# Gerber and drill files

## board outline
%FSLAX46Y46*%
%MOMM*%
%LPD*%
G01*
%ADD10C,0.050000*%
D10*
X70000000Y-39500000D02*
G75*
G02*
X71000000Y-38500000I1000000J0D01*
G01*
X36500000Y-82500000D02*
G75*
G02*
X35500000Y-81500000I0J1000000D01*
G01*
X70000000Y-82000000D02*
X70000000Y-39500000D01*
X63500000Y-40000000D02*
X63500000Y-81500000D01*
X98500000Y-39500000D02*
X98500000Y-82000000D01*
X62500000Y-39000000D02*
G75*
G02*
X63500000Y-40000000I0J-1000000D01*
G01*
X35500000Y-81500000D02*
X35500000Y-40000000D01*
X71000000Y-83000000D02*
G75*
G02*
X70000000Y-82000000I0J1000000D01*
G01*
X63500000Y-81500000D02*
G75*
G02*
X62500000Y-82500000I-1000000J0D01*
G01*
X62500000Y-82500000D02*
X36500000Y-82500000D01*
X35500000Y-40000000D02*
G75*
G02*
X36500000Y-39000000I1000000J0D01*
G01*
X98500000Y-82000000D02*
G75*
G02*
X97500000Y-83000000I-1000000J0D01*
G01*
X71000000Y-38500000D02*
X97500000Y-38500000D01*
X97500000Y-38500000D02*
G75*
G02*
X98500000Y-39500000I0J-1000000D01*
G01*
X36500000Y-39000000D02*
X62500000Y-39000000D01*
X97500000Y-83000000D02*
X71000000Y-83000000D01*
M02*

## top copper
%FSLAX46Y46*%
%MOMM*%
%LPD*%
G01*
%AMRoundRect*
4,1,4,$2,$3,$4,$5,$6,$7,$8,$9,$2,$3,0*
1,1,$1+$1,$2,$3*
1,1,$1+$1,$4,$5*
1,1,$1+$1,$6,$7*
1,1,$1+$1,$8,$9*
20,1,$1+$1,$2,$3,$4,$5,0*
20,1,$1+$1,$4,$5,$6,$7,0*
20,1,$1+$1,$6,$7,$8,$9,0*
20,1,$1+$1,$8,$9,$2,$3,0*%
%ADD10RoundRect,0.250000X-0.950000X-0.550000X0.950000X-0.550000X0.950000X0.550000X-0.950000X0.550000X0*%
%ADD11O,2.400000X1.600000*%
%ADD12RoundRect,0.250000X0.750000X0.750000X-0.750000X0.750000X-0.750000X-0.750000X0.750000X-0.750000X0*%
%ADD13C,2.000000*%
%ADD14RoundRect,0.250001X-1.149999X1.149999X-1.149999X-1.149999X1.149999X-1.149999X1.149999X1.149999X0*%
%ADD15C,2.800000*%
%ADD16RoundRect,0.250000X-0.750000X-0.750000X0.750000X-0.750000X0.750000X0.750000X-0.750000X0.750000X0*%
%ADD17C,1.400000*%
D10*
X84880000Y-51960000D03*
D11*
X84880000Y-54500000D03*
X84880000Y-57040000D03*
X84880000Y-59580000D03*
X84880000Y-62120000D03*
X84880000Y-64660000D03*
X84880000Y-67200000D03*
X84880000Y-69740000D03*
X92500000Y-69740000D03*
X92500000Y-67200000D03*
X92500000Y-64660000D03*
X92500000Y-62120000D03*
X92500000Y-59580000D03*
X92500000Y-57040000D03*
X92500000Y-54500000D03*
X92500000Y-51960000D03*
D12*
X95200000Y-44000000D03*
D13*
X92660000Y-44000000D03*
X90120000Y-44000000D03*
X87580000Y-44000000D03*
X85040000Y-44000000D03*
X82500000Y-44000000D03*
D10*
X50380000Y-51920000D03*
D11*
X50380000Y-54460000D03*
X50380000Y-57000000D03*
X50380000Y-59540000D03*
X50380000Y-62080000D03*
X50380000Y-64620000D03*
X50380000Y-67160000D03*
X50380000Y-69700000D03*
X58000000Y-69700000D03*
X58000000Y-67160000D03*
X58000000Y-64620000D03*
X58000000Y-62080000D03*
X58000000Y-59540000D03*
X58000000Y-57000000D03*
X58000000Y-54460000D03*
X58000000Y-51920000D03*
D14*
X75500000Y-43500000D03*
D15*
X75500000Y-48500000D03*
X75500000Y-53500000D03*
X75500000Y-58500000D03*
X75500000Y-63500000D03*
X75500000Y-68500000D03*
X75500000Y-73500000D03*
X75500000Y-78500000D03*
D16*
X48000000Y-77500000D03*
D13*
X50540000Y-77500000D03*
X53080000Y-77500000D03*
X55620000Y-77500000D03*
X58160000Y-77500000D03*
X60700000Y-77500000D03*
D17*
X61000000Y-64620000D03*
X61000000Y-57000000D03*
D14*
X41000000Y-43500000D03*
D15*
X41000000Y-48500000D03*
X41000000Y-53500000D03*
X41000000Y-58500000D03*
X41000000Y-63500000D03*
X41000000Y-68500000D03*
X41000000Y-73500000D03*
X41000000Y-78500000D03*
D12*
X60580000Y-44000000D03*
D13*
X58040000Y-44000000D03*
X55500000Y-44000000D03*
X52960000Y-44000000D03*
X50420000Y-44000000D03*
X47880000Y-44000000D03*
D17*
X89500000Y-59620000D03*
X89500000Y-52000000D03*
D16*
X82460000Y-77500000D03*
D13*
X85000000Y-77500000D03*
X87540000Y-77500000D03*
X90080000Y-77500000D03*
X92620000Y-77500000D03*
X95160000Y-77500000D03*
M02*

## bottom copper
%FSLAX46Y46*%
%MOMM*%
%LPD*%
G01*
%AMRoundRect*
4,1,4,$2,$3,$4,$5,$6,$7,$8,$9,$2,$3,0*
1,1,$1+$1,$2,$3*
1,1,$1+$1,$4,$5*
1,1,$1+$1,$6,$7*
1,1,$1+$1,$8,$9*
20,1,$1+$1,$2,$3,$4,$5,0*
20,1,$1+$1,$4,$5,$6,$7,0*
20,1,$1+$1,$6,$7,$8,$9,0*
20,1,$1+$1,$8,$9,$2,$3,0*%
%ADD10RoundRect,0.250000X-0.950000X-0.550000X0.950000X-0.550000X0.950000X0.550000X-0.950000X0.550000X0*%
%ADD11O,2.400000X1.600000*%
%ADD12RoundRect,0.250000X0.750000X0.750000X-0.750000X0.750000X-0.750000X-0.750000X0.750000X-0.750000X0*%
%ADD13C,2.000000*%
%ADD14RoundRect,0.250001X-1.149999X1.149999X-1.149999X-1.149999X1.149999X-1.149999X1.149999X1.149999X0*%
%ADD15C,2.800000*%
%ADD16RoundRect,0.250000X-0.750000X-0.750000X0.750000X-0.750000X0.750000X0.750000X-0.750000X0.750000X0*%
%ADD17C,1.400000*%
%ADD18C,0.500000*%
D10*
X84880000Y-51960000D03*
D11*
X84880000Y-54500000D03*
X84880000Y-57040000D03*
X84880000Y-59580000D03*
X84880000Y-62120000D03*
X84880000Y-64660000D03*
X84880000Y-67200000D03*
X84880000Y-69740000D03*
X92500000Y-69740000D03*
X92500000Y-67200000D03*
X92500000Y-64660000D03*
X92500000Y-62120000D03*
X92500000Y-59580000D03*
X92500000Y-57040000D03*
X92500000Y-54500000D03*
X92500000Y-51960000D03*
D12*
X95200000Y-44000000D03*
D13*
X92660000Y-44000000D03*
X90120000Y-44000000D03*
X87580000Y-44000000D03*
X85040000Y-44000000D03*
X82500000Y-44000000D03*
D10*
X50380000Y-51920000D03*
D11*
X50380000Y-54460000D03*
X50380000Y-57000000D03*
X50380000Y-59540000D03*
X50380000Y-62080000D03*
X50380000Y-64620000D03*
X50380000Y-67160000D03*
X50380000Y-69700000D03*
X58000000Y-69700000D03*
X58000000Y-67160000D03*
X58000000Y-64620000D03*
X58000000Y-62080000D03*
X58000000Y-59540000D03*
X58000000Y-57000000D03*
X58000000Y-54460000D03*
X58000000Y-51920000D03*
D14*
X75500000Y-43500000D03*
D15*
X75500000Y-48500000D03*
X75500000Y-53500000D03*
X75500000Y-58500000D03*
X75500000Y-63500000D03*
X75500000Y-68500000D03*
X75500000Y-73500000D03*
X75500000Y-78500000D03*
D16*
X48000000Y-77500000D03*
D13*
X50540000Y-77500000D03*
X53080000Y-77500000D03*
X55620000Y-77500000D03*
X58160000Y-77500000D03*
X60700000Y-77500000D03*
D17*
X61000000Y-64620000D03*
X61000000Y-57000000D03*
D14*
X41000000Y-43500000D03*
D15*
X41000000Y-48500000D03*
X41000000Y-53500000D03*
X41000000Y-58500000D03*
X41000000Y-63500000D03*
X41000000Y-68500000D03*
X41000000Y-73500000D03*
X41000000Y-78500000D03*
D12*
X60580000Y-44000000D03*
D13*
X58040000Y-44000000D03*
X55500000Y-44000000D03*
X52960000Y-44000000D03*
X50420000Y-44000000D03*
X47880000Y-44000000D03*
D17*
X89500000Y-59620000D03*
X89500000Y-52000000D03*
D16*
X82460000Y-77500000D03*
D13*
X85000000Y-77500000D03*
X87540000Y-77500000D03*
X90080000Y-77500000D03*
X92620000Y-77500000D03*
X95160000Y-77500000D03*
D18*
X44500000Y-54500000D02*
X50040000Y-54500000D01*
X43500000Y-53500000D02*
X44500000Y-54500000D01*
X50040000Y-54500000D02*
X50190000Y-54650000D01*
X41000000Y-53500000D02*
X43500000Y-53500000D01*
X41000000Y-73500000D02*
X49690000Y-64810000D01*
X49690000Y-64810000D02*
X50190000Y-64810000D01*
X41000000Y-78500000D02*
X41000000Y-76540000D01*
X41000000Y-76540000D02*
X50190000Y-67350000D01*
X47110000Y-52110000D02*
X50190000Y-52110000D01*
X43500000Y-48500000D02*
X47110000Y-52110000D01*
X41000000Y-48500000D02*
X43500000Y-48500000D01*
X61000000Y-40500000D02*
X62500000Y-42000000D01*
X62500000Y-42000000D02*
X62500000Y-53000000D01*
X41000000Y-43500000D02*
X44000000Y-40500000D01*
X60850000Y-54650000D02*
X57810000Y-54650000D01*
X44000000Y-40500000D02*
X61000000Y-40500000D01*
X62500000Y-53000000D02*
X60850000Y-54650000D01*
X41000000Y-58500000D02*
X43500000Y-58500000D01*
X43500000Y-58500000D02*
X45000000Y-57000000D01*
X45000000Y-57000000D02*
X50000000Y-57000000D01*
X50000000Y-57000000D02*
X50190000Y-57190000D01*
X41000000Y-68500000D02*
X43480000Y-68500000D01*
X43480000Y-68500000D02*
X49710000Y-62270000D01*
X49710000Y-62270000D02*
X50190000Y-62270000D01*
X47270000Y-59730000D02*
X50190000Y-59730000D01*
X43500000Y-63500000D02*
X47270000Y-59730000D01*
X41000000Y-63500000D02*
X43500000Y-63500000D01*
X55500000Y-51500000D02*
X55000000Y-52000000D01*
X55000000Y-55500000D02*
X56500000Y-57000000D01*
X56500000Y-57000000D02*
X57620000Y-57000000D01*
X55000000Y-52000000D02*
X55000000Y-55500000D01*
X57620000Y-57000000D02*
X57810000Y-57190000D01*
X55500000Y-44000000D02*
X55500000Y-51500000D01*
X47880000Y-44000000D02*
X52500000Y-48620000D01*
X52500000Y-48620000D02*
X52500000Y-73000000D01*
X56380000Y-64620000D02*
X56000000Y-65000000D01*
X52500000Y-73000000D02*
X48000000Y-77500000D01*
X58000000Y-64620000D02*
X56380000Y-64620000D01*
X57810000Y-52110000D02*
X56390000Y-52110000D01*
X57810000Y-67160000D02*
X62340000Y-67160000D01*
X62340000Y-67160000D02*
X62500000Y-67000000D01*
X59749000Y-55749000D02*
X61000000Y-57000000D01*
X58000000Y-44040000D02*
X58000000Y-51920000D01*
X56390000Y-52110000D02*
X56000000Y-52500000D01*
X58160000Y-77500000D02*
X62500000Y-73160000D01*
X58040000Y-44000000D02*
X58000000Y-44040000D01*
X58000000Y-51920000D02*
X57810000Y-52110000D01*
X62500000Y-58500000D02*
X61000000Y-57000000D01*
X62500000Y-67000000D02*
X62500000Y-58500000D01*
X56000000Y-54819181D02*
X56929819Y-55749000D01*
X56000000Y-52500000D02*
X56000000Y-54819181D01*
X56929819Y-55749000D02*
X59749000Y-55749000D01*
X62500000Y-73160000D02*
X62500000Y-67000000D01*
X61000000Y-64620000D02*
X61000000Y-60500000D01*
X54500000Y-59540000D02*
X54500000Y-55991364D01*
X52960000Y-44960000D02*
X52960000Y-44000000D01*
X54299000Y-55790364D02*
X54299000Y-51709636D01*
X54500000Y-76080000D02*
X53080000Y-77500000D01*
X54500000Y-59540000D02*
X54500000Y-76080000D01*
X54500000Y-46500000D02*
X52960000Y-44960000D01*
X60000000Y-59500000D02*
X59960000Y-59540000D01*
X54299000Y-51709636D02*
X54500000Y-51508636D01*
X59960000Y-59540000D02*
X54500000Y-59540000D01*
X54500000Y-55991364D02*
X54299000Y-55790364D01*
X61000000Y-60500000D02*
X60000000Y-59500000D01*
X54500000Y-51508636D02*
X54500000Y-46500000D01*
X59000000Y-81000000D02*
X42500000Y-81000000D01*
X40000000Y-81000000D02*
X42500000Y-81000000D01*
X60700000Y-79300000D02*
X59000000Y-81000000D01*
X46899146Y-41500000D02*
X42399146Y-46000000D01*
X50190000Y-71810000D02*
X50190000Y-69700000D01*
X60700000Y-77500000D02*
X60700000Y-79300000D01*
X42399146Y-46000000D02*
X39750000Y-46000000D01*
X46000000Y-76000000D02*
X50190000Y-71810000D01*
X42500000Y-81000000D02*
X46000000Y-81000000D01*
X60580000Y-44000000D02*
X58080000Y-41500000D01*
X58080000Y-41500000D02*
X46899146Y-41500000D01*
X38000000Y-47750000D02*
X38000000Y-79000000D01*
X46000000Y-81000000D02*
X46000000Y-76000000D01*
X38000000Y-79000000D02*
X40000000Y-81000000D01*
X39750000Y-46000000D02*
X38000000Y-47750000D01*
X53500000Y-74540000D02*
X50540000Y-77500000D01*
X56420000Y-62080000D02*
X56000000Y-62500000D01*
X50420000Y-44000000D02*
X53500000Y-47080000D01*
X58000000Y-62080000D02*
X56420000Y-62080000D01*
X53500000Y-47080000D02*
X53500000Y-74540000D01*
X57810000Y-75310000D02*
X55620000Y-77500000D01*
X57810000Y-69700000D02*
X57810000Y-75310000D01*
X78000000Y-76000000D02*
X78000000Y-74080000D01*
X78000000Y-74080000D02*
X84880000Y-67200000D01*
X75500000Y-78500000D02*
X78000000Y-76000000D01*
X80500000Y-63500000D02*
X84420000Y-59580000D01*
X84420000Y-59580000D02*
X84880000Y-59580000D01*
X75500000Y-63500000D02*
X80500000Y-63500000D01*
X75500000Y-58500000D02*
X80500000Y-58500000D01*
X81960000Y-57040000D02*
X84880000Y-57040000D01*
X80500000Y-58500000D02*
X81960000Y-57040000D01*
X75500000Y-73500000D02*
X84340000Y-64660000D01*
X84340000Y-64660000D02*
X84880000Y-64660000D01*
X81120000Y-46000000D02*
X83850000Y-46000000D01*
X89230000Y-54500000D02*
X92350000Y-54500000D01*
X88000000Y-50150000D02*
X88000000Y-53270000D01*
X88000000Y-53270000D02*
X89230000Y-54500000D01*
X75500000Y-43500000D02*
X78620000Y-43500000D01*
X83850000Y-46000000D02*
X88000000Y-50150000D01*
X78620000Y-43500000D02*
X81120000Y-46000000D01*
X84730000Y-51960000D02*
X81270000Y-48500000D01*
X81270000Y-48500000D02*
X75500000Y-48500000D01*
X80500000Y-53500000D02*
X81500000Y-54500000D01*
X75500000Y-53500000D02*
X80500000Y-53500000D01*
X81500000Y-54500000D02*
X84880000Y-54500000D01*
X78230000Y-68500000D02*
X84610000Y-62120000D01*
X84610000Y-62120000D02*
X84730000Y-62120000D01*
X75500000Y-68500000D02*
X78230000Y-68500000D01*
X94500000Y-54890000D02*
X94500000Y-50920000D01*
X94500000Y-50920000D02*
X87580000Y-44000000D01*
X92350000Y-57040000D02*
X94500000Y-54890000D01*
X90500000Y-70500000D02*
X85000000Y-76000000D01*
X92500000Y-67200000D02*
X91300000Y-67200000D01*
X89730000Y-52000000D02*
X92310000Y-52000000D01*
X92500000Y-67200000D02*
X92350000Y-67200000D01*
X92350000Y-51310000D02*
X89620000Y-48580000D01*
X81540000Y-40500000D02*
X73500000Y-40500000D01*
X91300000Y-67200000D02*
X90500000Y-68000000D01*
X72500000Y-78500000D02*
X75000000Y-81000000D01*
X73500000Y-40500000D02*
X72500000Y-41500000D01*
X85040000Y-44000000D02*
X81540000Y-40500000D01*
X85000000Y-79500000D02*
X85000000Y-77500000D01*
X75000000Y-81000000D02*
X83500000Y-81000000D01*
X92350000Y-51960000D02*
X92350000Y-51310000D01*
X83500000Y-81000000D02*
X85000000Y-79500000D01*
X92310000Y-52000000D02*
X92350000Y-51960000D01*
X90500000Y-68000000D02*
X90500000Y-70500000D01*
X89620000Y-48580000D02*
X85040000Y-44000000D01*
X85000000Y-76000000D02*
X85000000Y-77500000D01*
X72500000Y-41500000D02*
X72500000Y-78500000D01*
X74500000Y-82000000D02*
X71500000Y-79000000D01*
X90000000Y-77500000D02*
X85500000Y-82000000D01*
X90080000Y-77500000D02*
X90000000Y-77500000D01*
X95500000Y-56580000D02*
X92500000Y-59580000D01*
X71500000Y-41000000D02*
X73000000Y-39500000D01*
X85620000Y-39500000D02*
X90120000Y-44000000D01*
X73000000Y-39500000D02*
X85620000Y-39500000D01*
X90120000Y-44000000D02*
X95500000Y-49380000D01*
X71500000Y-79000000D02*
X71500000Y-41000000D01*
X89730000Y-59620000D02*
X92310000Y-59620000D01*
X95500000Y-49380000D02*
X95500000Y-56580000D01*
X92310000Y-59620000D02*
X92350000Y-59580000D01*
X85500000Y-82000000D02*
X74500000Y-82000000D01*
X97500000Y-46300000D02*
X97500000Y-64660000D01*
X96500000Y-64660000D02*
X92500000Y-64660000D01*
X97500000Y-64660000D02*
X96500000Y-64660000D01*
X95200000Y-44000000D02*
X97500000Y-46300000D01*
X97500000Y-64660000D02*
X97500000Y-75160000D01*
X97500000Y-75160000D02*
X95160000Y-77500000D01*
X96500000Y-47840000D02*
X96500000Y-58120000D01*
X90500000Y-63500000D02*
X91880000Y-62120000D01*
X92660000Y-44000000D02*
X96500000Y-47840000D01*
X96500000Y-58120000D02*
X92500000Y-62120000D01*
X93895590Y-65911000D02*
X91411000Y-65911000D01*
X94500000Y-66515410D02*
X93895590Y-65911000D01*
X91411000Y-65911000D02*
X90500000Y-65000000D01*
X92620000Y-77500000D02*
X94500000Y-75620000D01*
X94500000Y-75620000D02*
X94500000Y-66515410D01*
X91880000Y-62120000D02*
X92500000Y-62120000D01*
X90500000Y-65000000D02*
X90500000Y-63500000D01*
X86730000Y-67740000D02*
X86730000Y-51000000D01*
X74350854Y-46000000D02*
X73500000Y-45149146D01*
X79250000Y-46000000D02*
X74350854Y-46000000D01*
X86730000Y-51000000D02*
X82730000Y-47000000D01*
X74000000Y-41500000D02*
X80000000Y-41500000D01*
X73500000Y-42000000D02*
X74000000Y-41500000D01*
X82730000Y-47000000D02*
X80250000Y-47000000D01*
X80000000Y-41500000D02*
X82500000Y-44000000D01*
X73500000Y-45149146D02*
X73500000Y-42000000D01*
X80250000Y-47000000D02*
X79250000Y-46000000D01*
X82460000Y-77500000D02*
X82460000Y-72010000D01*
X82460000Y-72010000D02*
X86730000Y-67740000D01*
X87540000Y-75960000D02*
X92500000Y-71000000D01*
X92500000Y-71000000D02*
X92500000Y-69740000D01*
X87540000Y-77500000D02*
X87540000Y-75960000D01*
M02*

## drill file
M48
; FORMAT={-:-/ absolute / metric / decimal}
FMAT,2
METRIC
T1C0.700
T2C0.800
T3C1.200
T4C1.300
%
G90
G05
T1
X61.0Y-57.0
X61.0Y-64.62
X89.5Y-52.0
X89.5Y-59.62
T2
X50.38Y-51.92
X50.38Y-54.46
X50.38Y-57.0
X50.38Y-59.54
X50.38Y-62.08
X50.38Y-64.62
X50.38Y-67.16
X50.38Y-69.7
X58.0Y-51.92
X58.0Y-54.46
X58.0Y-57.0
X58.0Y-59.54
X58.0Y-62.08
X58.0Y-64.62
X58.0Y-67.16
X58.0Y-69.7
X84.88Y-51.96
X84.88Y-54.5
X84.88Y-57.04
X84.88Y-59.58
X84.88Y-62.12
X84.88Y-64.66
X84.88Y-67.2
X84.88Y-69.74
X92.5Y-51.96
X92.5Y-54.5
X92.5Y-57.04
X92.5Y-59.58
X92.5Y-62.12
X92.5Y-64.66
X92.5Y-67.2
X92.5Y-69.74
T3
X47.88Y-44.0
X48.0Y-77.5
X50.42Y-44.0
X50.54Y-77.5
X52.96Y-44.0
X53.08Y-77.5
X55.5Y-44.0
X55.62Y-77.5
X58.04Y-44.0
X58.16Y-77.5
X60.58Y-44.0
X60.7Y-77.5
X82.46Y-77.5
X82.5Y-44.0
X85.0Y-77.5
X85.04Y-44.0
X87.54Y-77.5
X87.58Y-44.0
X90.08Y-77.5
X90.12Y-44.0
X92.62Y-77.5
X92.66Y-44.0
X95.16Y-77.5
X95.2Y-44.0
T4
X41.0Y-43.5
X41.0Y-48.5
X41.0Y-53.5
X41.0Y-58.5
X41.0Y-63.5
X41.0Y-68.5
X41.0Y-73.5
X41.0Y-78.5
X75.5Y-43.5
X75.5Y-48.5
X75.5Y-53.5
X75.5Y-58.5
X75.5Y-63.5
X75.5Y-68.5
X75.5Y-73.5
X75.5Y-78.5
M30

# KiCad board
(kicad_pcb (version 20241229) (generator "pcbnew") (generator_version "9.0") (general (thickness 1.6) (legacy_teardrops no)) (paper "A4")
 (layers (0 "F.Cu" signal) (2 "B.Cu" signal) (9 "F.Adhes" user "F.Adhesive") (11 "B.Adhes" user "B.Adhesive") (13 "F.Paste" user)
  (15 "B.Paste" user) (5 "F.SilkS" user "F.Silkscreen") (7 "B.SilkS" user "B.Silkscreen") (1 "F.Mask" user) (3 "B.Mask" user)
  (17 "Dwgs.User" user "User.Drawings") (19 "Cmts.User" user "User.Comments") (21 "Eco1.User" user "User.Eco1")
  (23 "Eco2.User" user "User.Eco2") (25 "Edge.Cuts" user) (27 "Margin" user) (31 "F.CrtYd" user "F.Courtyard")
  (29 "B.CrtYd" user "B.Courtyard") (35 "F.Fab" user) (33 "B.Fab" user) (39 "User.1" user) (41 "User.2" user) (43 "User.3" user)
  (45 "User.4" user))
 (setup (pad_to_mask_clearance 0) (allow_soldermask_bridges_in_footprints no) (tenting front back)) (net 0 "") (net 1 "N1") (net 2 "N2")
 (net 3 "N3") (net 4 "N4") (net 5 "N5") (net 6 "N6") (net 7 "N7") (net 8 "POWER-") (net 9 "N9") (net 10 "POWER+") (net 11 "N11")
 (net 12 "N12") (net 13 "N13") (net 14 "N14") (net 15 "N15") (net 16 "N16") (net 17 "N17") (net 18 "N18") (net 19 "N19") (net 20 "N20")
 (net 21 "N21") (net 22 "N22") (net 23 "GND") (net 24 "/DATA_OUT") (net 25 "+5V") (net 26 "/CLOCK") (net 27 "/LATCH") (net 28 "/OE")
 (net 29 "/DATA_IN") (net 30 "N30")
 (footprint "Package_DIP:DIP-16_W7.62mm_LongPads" (layer "F.Cu") (at 84.88 51.96)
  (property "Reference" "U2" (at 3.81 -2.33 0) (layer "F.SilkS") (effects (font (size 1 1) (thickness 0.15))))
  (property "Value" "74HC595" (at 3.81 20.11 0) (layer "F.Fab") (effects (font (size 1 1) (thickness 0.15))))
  (pad "1" thru_hole roundrect (at 0 0) (size 2.4 1.6) (drill 0.8) (layers "*.Cu" "*.Mask") (remove_unused_layers no)
   (roundrect_rratio 0.15625) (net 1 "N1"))
  (pad "2" thru_hole oval (at 0 2.54) (size 2.4 1.6) (drill 0.8) (layers "*.Cu" "*.Mask") (remove_unused_layers no) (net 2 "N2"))
  (pad "3" thru_hole oval (at 0 5.08) (size 2.4 1.6) (drill 0.8) (layers "*.Cu" "*.Mask") (remove_unused_layers no) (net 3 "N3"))
  (pad "4" thru_hole oval (at 0 7.62) (size 2.4 1.6) (drill 0.8) (layers "*.Cu" "*.Mask") (remove_unused_layers no) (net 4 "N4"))
  (pad "5" thru_hole oval (at 0 10.16) (size 2.4 1.6) (drill 0.8) (layers "*.Cu" "*.Mask") (remove_unused_layers no) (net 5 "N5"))
  (pad "6" thru_hole oval (at 0 12.7) (size 2.4 1.6) (drill 0.8) (layers "*.Cu" "*.Mask") (remove_unused_layers no) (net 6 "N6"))
  (pad "7" thru_hole oval (at 0 15.24) (size 2.4 1.6) (drill 0.8) (layers "*.Cu" "*.Mask") (remove_unused_layers no) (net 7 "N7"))
  (pad "8" thru_hole oval (at 0 17.78) (size 2.4 1.6) (drill 0.8) (layers "*.Cu" "*.Mask") (remove_unused_layers no) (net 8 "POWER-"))
  (pad "9" thru_hole oval (at 7.62 17.78) (size 2.4 1.6) (drill 0.8) (layers "*.Cu" "*.Mask") (remove_unused_layers no) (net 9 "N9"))
  (pad "10" thru_hole oval (at 7.62 15.24) (size 2.4 1.6) (drill 0.8) (layers "*.Cu" "*.Mask") (remove_unused_layers no) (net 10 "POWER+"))
  (pad "11" thru_hole oval (at 7.62 12.7) (size 2.4 1.6) (drill 0.8) (layers "*.Cu" "*.Mask") (remove_unused_layers no) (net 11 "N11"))
  (pad "12" thru_hole oval (at 7.62 10.16) (size 2.4 1.6) (drill 0.8) (layers "*.Cu" "*.Mask") (remove_unused_layers no) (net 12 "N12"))
  (pad "13" thru_hole oval (at 7.62 7.62) (size 2.4 1.6) (drill 0.8) (layers "*.Cu" "*.Mask") (remove_unused_layers no) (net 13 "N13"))
  (pad "14" thru_hole oval (at 7.62 5.08) (size 2.4 1.6) (drill 0.8) (layers "*.Cu" "*.Mask") (remove_unused_layers no) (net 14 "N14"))
  (pad "15" thru_hole oval (at 7.62 2.54) (size 2.4 1.6) (drill 0.8) (layers "*.Cu" "*.Mask") (remove_unused_layers no) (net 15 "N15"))
  (pad "16" thru_hole oval (at 7.62 0) (size 2.4 1.6) (drill 0.8) (layers "*.Cu" "*.Mask") (remove_unused_layers no) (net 10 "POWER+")))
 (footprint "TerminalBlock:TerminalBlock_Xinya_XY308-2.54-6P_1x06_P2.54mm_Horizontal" (layer "F.Cu") (at 95.2 44 180)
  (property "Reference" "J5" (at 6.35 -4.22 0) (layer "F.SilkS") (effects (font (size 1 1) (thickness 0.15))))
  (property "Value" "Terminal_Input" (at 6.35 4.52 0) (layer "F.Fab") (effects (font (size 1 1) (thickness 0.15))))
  (pad "1" thru_hole roundrect (at 0 0 180) (size 2 2) (drill 1.2) (layers "*.Cu" "*.Mask") (remove_unused_layers no)
   (roundrect_rratio 0.125) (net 11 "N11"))
  (pad "2" thru_hole circle (at 2.54 0 180) (size 2 2) (drill 1.2) (layers "*.Cu" "*.Mask") (remove_unused_layers no) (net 12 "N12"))
  (pad "3" thru_hole circle (at 5.08 0 180) (size 2 2) (drill 1.2) (layers "*.Cu" "*.Mask") (remove_unused_layers no) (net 13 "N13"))
  (pad "4" thru_hole circle (at 7.62 0 180) (size 2 2) (drill 1.2) (layers "*.Cu" "*.Mask") (remove_unused_layers no) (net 14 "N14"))
  (pad "5" thru_hole circle (at 10.16 0 180) (size 2 2) (drill 1.2) (layers "*.Cu" "*.Mask") (remove_unused_layers no) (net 10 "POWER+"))
  (pad "6" thru_hole circle (at 12.7 0 180) (size 2 2) (drill 1.2) (layers "*.Cu" "*.Mask") (remove_unused_layers no) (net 8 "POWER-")))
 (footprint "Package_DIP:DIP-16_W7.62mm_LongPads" (layer "F.Cu") (at 50.38 51.92)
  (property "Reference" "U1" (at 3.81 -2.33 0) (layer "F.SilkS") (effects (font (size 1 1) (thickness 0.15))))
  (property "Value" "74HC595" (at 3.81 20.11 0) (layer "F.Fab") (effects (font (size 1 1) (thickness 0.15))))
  (pad "1" thru_hole roundrect (at 0 0) (size 2.4 1.6) (drill 0.8) (layers "*.Cu" "*.Mask") (remove_unused_layers no)
   (roundrect_rratio 0.15625) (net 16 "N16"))
  (pad "2" thru_hole oval (at 0 2.54) (size 2.4 1.6) (drill 0.8) (layers "*.Cu" "*.Mask") (remove_unused_layers no) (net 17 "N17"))
  (pad "3" thru_hole oval (at 0 5.08) (size 2.4 1.6) (drill 0.8) (layers "*.Cu" "*.Mask") (remove_unused_layers no) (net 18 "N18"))
  (pad "4" thru_hole oval (at 0 7.62) (size 2.4 1.6) (drill 0.8) (layers "*.Cu" "*.Mask") (remove_unused_layers no) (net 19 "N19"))
  (pad "5" thru_hole oval (at 0 10.16) (size 2.4 1.6) (drill 0.8) (layers "*.Cu" "*.Mask") (remove_unused_layers no) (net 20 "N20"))
  (pad "6" thru_hole oval (at 0 12.7) (size 2.4 1.6) (drill 0.8) (layers "*.Cu" "*.Mask") (remove_unused_layers no) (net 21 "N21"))
  (pad "7" thru_hole oval (at 0 15.24) (size 2.4 1.6) (drill 0.8) (layers "*.Cu" "*.Mask") (remove_unused_layers no) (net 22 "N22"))
  (pad "8" thru_hole oval (at 0 17.78) (size 2.4 1.6) (drill 0.8) (layers "*.Cu" "*.Mask") (remove_unused_layers no) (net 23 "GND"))
  (pad "9" thru_hole oval (at 7.62 17.78) (size 2.4 1.6) (drill 0.8) (layers "*.Cu" "*.Mask") (remove_unused_layers no) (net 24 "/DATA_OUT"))
  (pad "10" thru_hole oval (at 7.62 15.24) (size 2.4 1.6) (drill 0.8) (layers "*.Cu" "*.Mask") (remove_unused_layers no) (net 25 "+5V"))
  (pad "11" thru_hole oval (at 7.62 12.7) (size 2.4 1.6) (drill 0.8) (layers "*.Cu" "*.Mask") (remove_unused_layers no) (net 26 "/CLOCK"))
  (pad "12" thru_hole oval (at 7.62 10.16) (size 2.4 1.6) (drill 0.8) (layers "*.Cu" "*.Mask") (remove_unused_layers no) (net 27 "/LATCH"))
  (pad "13" thru_hole oval (at 7.62 7.62) (size 2.4 1.6) (drill 0.8) (layers "*.Cu" "*.Mask") (remove_unused_layers no) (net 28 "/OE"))
  (pad "14" thru_hole oval (at 7.62 5.08) (size 2.4 1.6) (drill 0.8) (layers "*.Cu" "*.Mask") (remove_unused_layers no) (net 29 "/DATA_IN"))
  (pad "15" thru_hole oval (at 7.62 2.54) (size 2.4 1.6) (drill 0.8) (layers "*.Cu" "*.Mask") (remove_unused_layers no) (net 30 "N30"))
  (pad "16" thru_hole oval (at 7.62 0) (size 2.4 1.6) (drill 0.8) (layers "*.Cu" "*.Mask") (remove_unused_layers no) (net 25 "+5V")))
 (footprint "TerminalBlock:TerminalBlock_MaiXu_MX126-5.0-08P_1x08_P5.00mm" (layer "F.Cu") (at 75.5 43.5 -90)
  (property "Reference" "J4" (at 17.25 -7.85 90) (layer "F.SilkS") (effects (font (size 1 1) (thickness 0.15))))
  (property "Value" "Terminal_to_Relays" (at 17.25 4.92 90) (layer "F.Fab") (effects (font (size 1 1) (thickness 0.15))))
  (pad "1" thru_hole roundrect (at 0 0 270) (size 2.8 2.8) (drill 1.3) (layers "*.Cu" "*.Mask") (remove_unused_layers no)
   (roundrect_rratio 0.089286) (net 15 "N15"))
  (pad "2" thru_hole circle (at 5 0 270) (size 2.8 2.8) (drill 1.3) (layers "*.Cu" "*.Mask") (remove_unused_layers no) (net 1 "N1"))
  (pad "3" thru_hole circle (at 10 0 270) (size 2.8 2.8) (drill 1.3) (layers "*.Cu" "*.Mask") (remove_unused_layers no) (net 2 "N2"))
  (pad "4" thru_hole circle (at 15 0 270) (size 2.8 2.8) (drill 1.3) (layers "*.Cu" "*.Mask") (remove_unused_layers no) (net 3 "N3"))
  (pad "5" thru_hole circle (at 20 0 270) (size 2.8 2.8) (drill 1.3) (layers "*.Cu" "*.Mask") (remove_unused_layers no) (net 4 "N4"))
  (pad "6" thru_hole circle (at 25 0 270) (size 2.8 2.8) (drill 1.3) (layers "*.Cu" "*.Mask") (remove_unused_layers no) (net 5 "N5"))
  (pad "7" thru_hole circle (at 30 0 270) (size 2.8 2.8) (drill 1.3) (layers "*.Cu" "*.Mask") (remove_unused_layers no) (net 6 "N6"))
  (pad "8" thru_hole circle (at 35 0 270) (size 2.8 2.8) (drill 1.3) (layers "*.Cu" "*.Mask") (remove_unused_layers no) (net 7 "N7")))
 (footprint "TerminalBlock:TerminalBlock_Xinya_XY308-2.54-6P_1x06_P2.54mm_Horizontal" (layer "F.Cu") (at 48 77.5)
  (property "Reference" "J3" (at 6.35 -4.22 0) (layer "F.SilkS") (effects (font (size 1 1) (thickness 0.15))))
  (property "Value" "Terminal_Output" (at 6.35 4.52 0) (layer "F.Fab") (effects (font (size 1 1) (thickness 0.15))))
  (pad "1" thru_hole roundrect (at 0 0) (size 2 2) (drill 1.2) (layers "*.Cu" "*.Mask") (remove_unused_layers no) (roundrect_rratio 0.125)
   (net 26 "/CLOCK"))
  (pad "2" thru_hole circle (at 2.54 0) (size 2 2) (drill 1.2) (layers "*.Cu" "*.Mask") (remove_unused_layers no) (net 27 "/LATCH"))
  (pad "3" thru_hole circle (at 5.08 0) (size 2 2) (drill 1.2) (layers "*.Cu" "*.Mask") (remove_unused_layers no) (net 28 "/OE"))
  (pad "4" thru_hole circle (at 7.62 0) (size 2 2) (drill 1.2) (layers "*.Cu" "*.Mask") (remove_unused_layers no) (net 24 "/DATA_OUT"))
  (pad "5" thru_hole circle (at 10.16 0) (size 2 2) (drill 1.2) (layers "*.Cu" "*.Mask") (remove_unused_layers no) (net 25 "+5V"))
  (pad "6" thru_hole circle (at 12.7 0) (size 2 2) (drill 1.2) (layers "*.Cu" "*.Mask") (remove_unused_layers no) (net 23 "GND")))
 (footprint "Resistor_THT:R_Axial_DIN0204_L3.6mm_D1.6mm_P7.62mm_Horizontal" (layer "F.Cu") (at 61 64.62 90)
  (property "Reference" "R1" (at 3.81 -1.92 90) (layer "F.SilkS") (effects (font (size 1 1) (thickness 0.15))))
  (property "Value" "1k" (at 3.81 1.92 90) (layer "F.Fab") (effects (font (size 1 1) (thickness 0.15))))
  (pad "1" thru_hole circle (at 0 0 90) (size 1.4 1.4) (drill 0.7) (layers "*.Cu" "*.Mask") (remove_unused_layers no) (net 28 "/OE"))
  (pad "2" thru_hole circle (at 7.62 0 90) (size 1.4 1.4) (drill 0.7) (layers "*.Cu" "*.Mask") (remove_unused_layers no) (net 25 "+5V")))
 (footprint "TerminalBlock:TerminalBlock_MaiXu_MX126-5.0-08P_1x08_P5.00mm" (layer "F.Cu") (at 41 43.5 -90)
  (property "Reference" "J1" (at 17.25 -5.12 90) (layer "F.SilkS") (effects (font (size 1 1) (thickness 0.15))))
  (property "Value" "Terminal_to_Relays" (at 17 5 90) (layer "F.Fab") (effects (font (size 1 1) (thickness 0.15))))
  (pad "1" thru_hole roundrect (at 0 0 270) (size 2.8 2.8) (drill 1.3) (layers "*.Cu" "*.Mask") (remove_unused_layers no)
   (roundrect_rratio 0.089286) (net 30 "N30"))
  (pad "2" thru_hole circle (at 5 0 270) (size 2.8 2.8) (drill 1.3) (layers "*.Cu" "*.Mask") (remove_unused_layers no) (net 16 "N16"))
  (pad "3" thru_hole circle (at 10 0 270) (size 2.8 2.8) (drill 1.3) (layers "*.Cu" "*.Mask") (remove_unused_layers no) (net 17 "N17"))
  (pad "4" thru_hole circle (at 15 0 270) (size 2.8 2.8) (drill 1.3) (layers "*.Cu" "*.Mask") (remove_unused_layers no) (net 18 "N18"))
  (pad "5" thru_hole circle (at 20 0 270) (size 2.8 2.8) (drill 1.3) (layers "*.Cu" "*.Mask") (remove_unused_layers no) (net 19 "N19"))
  (pad "6" thru_hole circle (at 25 0 270) (size 2.8 2.8) (drill 1.3) (layers "*.Cu" "*.Mask") (remove_unused_layers no) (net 20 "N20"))
  (pad "7" thru_hole circle (at 30 0 270) (size 2.8 2.8) (drill 1.3) (layers "*.Cu" "*.Mask") (remove_unused_layers no) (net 21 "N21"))
  (pad "8" thru_hole circle (at 35 0 270) (size 2.8 2.8) (drill 1.3) (layers "*.Cu" "*.Mask") (remove_unused_layers no) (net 22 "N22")))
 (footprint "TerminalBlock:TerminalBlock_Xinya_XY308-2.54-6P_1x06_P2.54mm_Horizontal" (layer "F.Cu") (at 60.58 44 180)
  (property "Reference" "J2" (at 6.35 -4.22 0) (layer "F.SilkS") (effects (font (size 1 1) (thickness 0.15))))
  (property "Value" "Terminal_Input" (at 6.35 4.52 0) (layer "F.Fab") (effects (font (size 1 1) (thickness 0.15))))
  (pad "1" thru_hole roundrect (at 0 0 180) (size 2 2) (drill 1.2) (layers "*.Cu" "*.Mask") (remove_unused_layers no)
   (roundrect_rratio 0.125) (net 23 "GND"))
  (pad "2" thru_hole circle (at 2.54 0 180) (size 2 2) (drill 1.2) (layers "*.Cu" "*.Mask") (remove_unused_layers no) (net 25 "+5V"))
  (pad "3" thru_hole circle (at 5.08 0 180) (size 2 2) (drill 1.2) (layers "*.Cu" "*.Mask") (remove_unused_layers no) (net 29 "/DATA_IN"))
  (pad "4" thru_hole circle (at 7.62 0 180) (size 2 2) (drill 1.2) (layers "*.Cu" "*.Mask") (remove_unused_layers no) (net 28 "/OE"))
  (pad "5" thru_hole circle (at 10.16 0 180) (size 2 2) (drill 1.2) (layers "*.Cu" "*.Mask") (remove_unused_layers no) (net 27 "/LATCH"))
  (pad "6" thru_hole circle (at 12.7 0 180) (size 2 2) (drill 1.2) (layers "*.Cu" "*.Mask") (remove_unused_layers no) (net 26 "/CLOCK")))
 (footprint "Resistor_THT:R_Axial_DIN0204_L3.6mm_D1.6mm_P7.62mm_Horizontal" (layer "F.Cu") (at 89.5 59.62 90)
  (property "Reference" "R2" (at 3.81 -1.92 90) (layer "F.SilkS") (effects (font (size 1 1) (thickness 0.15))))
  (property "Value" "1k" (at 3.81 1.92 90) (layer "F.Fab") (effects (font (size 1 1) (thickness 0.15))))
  (pad "1" thru_hole circle (at 0 0 90) (size 1.4 1.4) (drill 0.7) (layers "*.Cu" "*.Mask") (remove_unused_layers no) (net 13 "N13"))
  (pad "2" thru_hole circle (at 7.62 0 90) (size 1.4 1.4) (drill 0.7) (layers "*.Cu" "*.Mask") (remove_unused_layers no) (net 10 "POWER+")))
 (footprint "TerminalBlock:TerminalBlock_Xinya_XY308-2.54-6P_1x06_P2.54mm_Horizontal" (layer "F.Cu") (at 82.46 77.5)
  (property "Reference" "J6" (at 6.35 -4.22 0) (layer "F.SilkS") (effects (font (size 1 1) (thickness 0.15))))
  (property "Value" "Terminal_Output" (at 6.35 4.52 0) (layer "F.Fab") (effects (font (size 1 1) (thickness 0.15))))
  (pad "1" thru_hole roundrect (at 0 0) (size 2 2) (drill 1.2) (layers "*.Cu" "*.Mask") (remove_unused_layers no) (roundrect_rratio 0.125)
   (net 8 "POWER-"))
  (pad "2" thru_hole circle (at 2.54 0) (size 2 2) (drill 1.2) (layers "*.Cu" "*.Mask") (remove_unused_layers no) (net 10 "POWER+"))
  (pad "3" thru_hole circle (at 5.08 0) (size 2 2) (drill 1.2) (layers "*.Cu" "*.Mask") (remove_unused_layers no) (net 9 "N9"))
  (pad "4" thru_hole circle (at 7.62 0) (size 2 2) (drill 1.2) (layers "*.Cu" "*.Mask") (remove_unused_layers no) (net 13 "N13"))
  (pad "5" thru_hole circle (at 10.16 0) (size 2 2) (drill 1.2) (layers "*.Cu" "*.Mask") (remove_unused_layers no) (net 12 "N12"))
  (pad "6" thru_hole circle (at 12.7 0) (size 2 2) (drill 1.2) (layers "*.Cu" "*.Mask") (remove_unused_layers no) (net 11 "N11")))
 (gr_arc (start 70 39.5) (mid 70.292893 38.792893) (end 71 38.5) (stroke (width 0.05) (type default)) (layer "Edge.Cuts"))
 (gr_arc (start 36.5 82.5) (mid 35.792893 82.207107) (end 35.5 81.5) (stroke (width 0.05) (type default)) (layer "Edge.Cuts"))
 (gr_line (start 70 82) (end 70 39.5) (stroke (width 0.05) (type default)) (layer "Edge.Cuts"))
 (gr_line (start 63.5 40) (end 63.5 81.5) (stroke (width 0.05) (type default)) (layer "Edge.Cuts"))
 (gr_line (start 98.5 39.5) (end 98.5 82) (stroke (width 0.05) (type default)) (layer "Edge.Cuts"))
 (gr_arc (start 62.5 39) (mid 63.207107 39.292893) (end 63.5 40) (stroke (width 0.05) (type default)) (layer "Edge.Cuts"))
 (gr_line (start 35.5 81.5) (end 35.5 40) (stroke (width 0.05) (type default)) (layer "Edge.Cuts"))
 (gr_arc (start 71 83) (mid 70.292893 82.707107) (end 70 82) (stroke (width 0.05) (type default)) (layer "Edge.Cuts"))
 (gr_arc (start 63.5 81.5) (mid 63.207107 82.207107) (end 62.5 82.5) (stroke (width 0.05) (type default)) (layer "Edge.Cuts"))
 (gr_line (start 62.5 82.5) (end 36.5 82.5) (stroke (width 0.05) (type default)) (layer "Edge.Cuts"))
 (gr_arc (start 35.5 40) (mid 35.792893 39.292893) (end 36.5 39) (stroke (width 0.05) (type default)) (layer "Edge.Cuts"))
 (gr_arc (start 98.5 82) (mid 98.207107 82.707107) (end 97.5 83) (stroke (width 0.05) (type default)) (layer "Edge.Cuts"))
 (gr_line (start 71 38.5) (end 97.5 38.5) (stroke (width 0.05) (type default)) (layer "Edge.Cuts"))
 (gr_arc (start 97.5 38.5) (mid 98.207107 38.792893) (end 98.5 39.5) (stroke (width 0.05) (type default)) (layer "Edge.Cuts"))
 (gr_line (start 36.5 39) (end 62.5 39) (stroke (width 0.05) (type default)) (layer "Edge.Cuts"))
 (gr_line (start 97.5 83) (end 71 83) (stroke (width 0.05) (type default)) (layer "Edge.Cuts"))
 (segment (start 44.5 54.5) (end 50.04 54.5) (width 0.5) (layer "B.Cu") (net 17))
 (segment (start 43.5 53.5) (end 44.5 54.5) (width 0.5) (layer "B.Cu") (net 17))
 (segment (start 50.04 54.5) (end 50.19 54.65) (width 0.5) (layer "B.Cu") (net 17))
 (segment (start 41 53.5) (end 43.5 53.5) (width 0.5) (layer "B.Cu") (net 17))
 (segment (start 41 73.5) (end 49.69 64.81) (width 0.5) (layer "B.Cu") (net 21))
 (segment (start 49.69 64.81) (end 50.19 64.81) (width 0.5) (layer "B.Cu") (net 21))
 (segment (start 41 78.5) (end 41 76.54) (width 0.5) (layer "B.Cu") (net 22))
 (segment (start 41 76.54) (end 50.19 67.35) (width 0.5) (layer "B.Cu") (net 22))
 (segment (start 47.11 52.11) (end 50.19 52.11) (width 0.5) (layer "B.Cu") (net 16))
 (segment (start 43.5 48.5) (end 47.11 52.11) (width 0.5) (layer "B.Cu") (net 16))
 (segment (start 41 48.5) (end 43.5 48.5) (width 0.5) (layer "B.Cu") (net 16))
 (segment (start 61 40.5) (end 62.5 42) (width 0.5) (layer "B.Cu") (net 30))
 (segment (start 62.5 42) (end 62.5 53) (width 0.5) (layer "B.Cu") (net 30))
 (segment (start 41 43.5) (end 44 40.5) (width 0.5) (layer "B.Cu") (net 30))
 (segment (start 60.85 54.65) (end 57.81 54.65) (width 0.5) (layer "B.Cu") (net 30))
 (segment (start 44 40.5) (end 61 40.5) (width 0.5) (layer "B.Cu") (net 30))
 (segment (start 62.5 53) (end 60.85 54.65) (width 0.5) (layer "B.Cu") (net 30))
 (segment (start 41 58.5) (end 43.5 58.5) (width 0.5) (layer "B.Cu") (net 18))
 (segment (start 43.5 58.5) (end 45 57) (width 0.5) (layer "B.Cu") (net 18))
 (segment (start 45 57) (end 50 57) (width 0.5) (layer "B.Cu") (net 18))
 (segment (start 50 57) (end 50.19 57.19) (width 0.5) (layer "B.Cu") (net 18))
 (segment (start 41 68.5) (end 43.48 68.5) (width 0.5) (layer "B.Cu") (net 20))
 (segment (start 43.48 68.5) (end 49.71 62.27) (width 0.5) (layer "B.Cu") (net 20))
 (segment (start 49.71 62.27) (end 50.19 62.27) (width 0.5) (layer "B.Cu") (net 20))
 (segment (start 47.27 59.73) (end 50.19 59.73) (width 0.5) (layer "B.Cu") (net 19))
 (segment (start 43.5 63.5) (end 47.27 59.73) (width 0.5) (layer "B.Cu") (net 19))
 (segment (start 41 63.5) (end 43.5 63.5) (width 0.5) (layer "B.Cu") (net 19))
 (segment (start 55.5 51.5) (end 55 52) (width 0.5) (layer "B.Cu") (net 29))
 (segment (start 55 55.5) (end 56.5 57) (width 0.5) (layer "B.Cu") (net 29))
 (segment (start 56.5 57) (end 57.62 57) (width 0.5) (layer "B.Cu") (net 29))
 (segment (start 55 52) (end 55 55.5) (width 0.5) (layer "B.Cu") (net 29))
 (segment (start 57.62 57) (end 57.81 57.19) (width 0.5) (layer "B.Cu") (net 29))
 (segment (start 55.5 44) (end 55.5 51.5) (width 0.5) (layer "B.Cu") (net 29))
 (segment (start 47.88 44) (end 52.5 48.62) (width 0.5) (layer "B.Cu") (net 26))
 (segment (start 52.5 48.62) (end 52.5 73) (width 0.5) (layer "B.Cu") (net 26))
 (segment (start 56.38 64.62) (end 56 65) (width 0.5) (layer "B.Cu") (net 26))
 (segment (start 52.5 73) (end 48 77.5) (width 0.5) (layer "B.Cu") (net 26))
 (segment (start 58 64.62) (end 56.38 64.62) (width 0.5) (layer "B.Cu") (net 26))
 (segment (start 57.81 52.11) (end 56.39 52.11) (width 0.5) (layer "B.Cu") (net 25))
 (segment (start 57.81 67.16) (end 62.34 67.16) (width 0.5) (layer "B.Cu") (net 25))
 (segment (start 62.34 67.16) (end 62.5 67) (width 0.5) (layer "B.Cu") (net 25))
 (segment (start 59.749 55.749) (end 61 57) (width 0.5) (layer "B.Cu") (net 25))
 (segment (start 58 44.04) (end 58 51.92) (width 0.5) (layer "B.Cu") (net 25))
 (segment (start 56.39 52.11) (end 56 52.5) (width 0.5) (layer "B.Cu") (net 25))
 (segment (start 58.16 77.5) (end 62.5 73.16) (width 0.5) (layer "B.Cu") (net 25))
 (segment (start 58.04 44) (end 58 44.04) (width 0.5) (layer "B.Cu") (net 25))
 (segment (start 58 51.92) (end 57.81 52.11) (width 0.5) (layer "B.Cu") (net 25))
 (segment (start 62.5 58.5) (end 61 57) (width 0.5) (layer "B.Cu") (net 25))
 (segment (start 62.5 67) (end 62.5 58.5) (width 0.5) (layer "B.Cu") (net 25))
 (segment (start 56 54.819181) (end 56.929819 55.749) (width 0.5) (layer "B.Cu") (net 25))
 (segment (start 56 52.5) (end 56 54.819181) (width 0.5) (layer "B.Cu") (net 25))
 (segment (start 56.929819 55.749) (end 59.749 55.749) (width 0.5) (layer "B.Cu") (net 25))
 (segment (start 62.5 73.16) (end 62.5 67) (width 0.5) (layer "B.Cu") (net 25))
 (segment (start 61 64.62) (end 61 60.5) (width 0.5) (layer "B.Cu") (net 28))
 (segment (start 54.5 59.54) (end 54.5 55.991364) (width 0.5) (layer "B.Cu") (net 28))
 (segment (start 52.96 44.96) (end 52.96 44) (width 0.5) (layer "B.Cu") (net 28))
 (segment (start 54.299 55.790364) (end 54.299 51.709636) (width 0.5) (layer "B.Cu") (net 28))
 (segment (start 54.5 76.08) (end 53.08 77.5) (width 0.5) (layer "B.Cu") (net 28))
 (segment (start 54.5 59.54) (end 54.5 76.08) (width 0.5) (layer "B.Cu") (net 28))
 (segment (start 54.5 46.5) (end 52.96 44.96) (width 0.5) (layer "B.Cu") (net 28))
 (segment (start 60 59.5) (end 59.96 59.54) (width 0.5) (layer "B.Cu") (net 28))
 (segment (start 54.299 51.709636) (end 54.5 51.508636) (width 0.5) (layer "B.Cu") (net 28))
 (segment (start 59.96 59.54) (end 54.5 59.54) (width 0.5) (layer "B.Cu") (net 28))
 (segment (start 54.5 55.991364) (end 54.299 55.790364) (width 0.5) (layer "B.Cu") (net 28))
 (segment (start 61 60.5) (end 60 59.5) (width 0.5) (layer "B.Cu") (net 28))
 (segment (start 54.5 51.508636) (end 54.5 46.5) (width 0.5) (layer "B.Cu") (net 28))
 (segment (start 59 81) (end 42.5 81) (width 0.5) (layer "B.Cu") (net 23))
 (segment (start 40 81) (end 42.5 81) (width 0.5) (layer "B.Cu") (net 23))
 (segment (start 60.7 79.3) (end 59 81) (width 0.5) (layer "B.Cu") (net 23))
 (segment (start 46.899146 41.5) (end 42.399146 46) (width 0.5) (layer "B.Cu") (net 23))
 (segment (start 50.19 71.81) (end 50.19 69.7) (width 0.5) (layer "B.Cu") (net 23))
 (segment (start 60.7 77.5) (end 60.7 79.3) (width 0.5) (layer "B.Cu") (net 23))
 (segment (start 42.399146 46) (end 39.75 46) (width 0.5) (layer "B.Cu") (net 23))
 (segment (start 46 76) (end 50.19 71.81) (width 0.5) (layer "B.Cu") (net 23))
 (segment (start 42.5 81) (end 46 81) (width 0.5) (layer "B.Cu") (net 23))
 (segment (start 60.58 44) (end 58.08 41.5) (width 0.5) (layer "B.Cu") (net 23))
 (segment (start 58.08 41.5) (end 46.899146 41.5) (width 0.5) (layer "B.Cu") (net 23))
 (segment (start 38 47.75) (end 38 79) (width 0.5) (layer "B.Cu") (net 23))
 (segment (start 46 81) (end 46 76) (width 0.5) (layer "B.Cu") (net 23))
 (segment (start 38 79) (end 40 81) (width 0.5) (layer "B.Cu") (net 23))
 (segment (start 39.75 46) (end 38 47.75) (width 0.5) (layer "B.Cu") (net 23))
 (segment (start 53.5 74.54) (end 50.54 77.5) (width 0.5) (layer "B.Cu") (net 27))
 (segment (start 56.42 62.08) (end 56 62.5) (width 0.5) (layer "B.Cu") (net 27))
 (segment (start 50.42 44) (end 53.5 47.08) (width 0.5) (layer "B.Cu") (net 27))
 (segment (start 58 62.08) (end 56.42 62.08) (width 0.5) (layer "B.Cu") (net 27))
 (segment (start 53.5 47.08) (end 53.5 74.54) (width 0.5) (layer "B.Cu") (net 27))
 (segment (start 57.81 75.31) (end 55.62 77.5) (width 0.5) (layer "B.Cu") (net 24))
 (segment (start 57.81 69.7) (end 57.81 75.31) (width 0.5) (layer "B.Cu") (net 24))
 (segment (start 78 76) (end 78 74.08) (width 0.5) (layer "B.Cu") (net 7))
 (segment (start 78 74.08) (end 84.88 67.2) (width 0.5) (layer "B.Cu") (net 7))
 (segment (start 75.5 78.5) (end 78 76) (width 0.5) (layer "B.Cu") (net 7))
 (segment (start 80.5 63.5) (end 84.42 59.58) (width 0.5) (layer "B.Cu") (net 4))
 (segment (start 84.42 59.58) (end 84.88 59.58) (width 0.5) (layer "B.Cu") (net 4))
 (segment (start 75.5 63.5) (end 80.5 63.5) (width 0.5) (layer "B.Cu") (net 4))
 (segment (start 75.5 58.5) (end 80.5 58.5) (width 0.5) (layer "B.Cu") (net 3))
 (segment (start 81.96 57.04) (end 84.88 57.04) (width 0.5) (layer "B.Cu") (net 3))
 (segment (start 80.5 58.5) (end 81.96 57.04) (width 0.5) (layer "B.Cu") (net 3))
 (segment (start 75.5 73.5) (end 84.34 64.66) (width 0.5) (layer "B.Cu") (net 6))
 (segment (start 84.34 64.66) (end 84.88 64.66) (width 0.5) (layer "B.Cu") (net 6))
 (segment (start 81.12 46) (end 83.85 46) (width 0.5) (layer "B.Cu") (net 15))
 (segment (start 89.23 54.5) (end 92.35 54.5) (width 0.5) (layer "B.Cu") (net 15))
 (segment (start 88 50.15) (end 88 53.27) (width 0.5) (layer "B.Cu") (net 15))
 (segment (start 88 53.27) (end 89.23 54.5) (width 0.5) (layer "B.Cu") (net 15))
 (segment (start 75.5 43.5) (end 78.62 43.5) (width 0.5) (layer "B.Cu") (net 15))
 (segment (start 83.85 46) (end 88 50.15) (width 0.5) (layer "B.Cu") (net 15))
 (segment (start 78.62 43.5) (end 81.12 46) (width 0.5) (layer "B.Cu") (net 15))
 (segment (start 84.73 51.96) (end 81.27 48.5) (width 0.5) (layer "B.Cu") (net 1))
 (segment (start 81.27 48.5) (end 75.5 48.5) (width 0.5) (layer "B.Cu") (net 1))
 (segment (start 80.5 53.5) (end 81.5 54.5) (width 0.5) (layer "B.Cu") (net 2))
 (segment (start 75.5 53.5) (end 80.5 53.5) (width 0.5) (layer "B.Cu") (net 2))
 (segment (start 81.5 54.5) (end 84.88 54.5) (width 0.5) (layer "B.Cu") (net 2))
 (segment (start 78.23 68.5) (end 84.61 62.12) (width 0.5) (layer "B.Cu") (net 5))
 (segment (start 84.61 62.12) (end 84.73 62.12) (width 0.5) (layer "B.Cu") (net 5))
 (segment (start 75.5 68.5) (end 78.23 68.5) (width 0.5) (layer "B.Cu") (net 5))
 (segment (start 94.5 54.89) (end 94.5 50.92) (width 0.5) (layer "B.Cu") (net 14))
 (segment (start 94.5 50.92) (end 87.58 44) (width 0.5) (layer "B.Cu") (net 14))
 (segment (start 92.35 57.04) (end 94.5 54.89) (width 0.5) (layer "B.Cu") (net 14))
 (segment (start 90.5 70.5) (end 85 76) (width 0.5) (layer "B.Cu") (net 10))
 (segment (start 92.5 67.2) (end 91.3 67.2) (width 0.5) (layer "B.Cu") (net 10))
 (segment (start 89.73 52) (end 92.31 52) (width 0.5) (layer "B.Cu") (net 10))
 (segment (start 92.5 67.2) (end 92.35 67.2) (width 0.5) (layer "B.Cu") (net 10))
 (segment (start 92.35 51.31) (end 89.62 48.58) (width 0.5) (layer "B.Cu") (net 10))
 (segment (start 81.54 40.5) (end 73.5 40.5) (width 0.5) (layer "B.Cu") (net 10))
 (segment (start 91.3 67.2) (end 90.5 68) (width 0.5) (layer "B.Cu") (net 10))
 (segment (start 72.5 78.5) (end 75 81) (width 0.5) (layer "B.Cu") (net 10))
 (segment (start 73.5 40.5) (end 72.5 41.5) (width 0.5) (layer "B.Cu") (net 10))
 (segment (start 85.04 44) (end 81.54 40.5) (width 0.5) (layer "B.Cu") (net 10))
 (segment (start 85 79.5) (end 85 77.5) (width 0.5) (layer "B.Cu") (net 10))
 (segment (start 75 81) (end 83.5 81) (width 0.5) (layer "B.Cu") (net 10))
 (segment (start 92.35 51.96) (end 92.35 51.31) (width 0.5) (layer "B.Cu") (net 10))
 (segment (start 83.5 81) (end 85 79.5) (width 0.5) (layer "B.Cu") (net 10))
 (segment (start 92.31 52) (end 92.35 51.96) (width 0.5) (layer "B.Cu") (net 10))
 (segment (start 90.5 68) (end 90.5 70.5) (width 0.5) (layer "B.Cu") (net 10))
 (segment (start 89.62 48.58) (end 85.04 44) (width 0.5) (layer "B.Cu") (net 10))
 (segment (start 85 76) (end 85 77.5) (width 0.5) (layer "B.Cu") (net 10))
 (segment (start 72.5 41.5) (end 72.5 78.5) (width 0.5) (layer "B.Cu") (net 10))
 (segment (start 74.5 82) (end 71.5 79) (width 0.5) (layer "B.Cu") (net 13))
 (segment (start 90 77.5) (end 85.5 82) (width 0.5) (layer "B.Cu") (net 13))
 (segment (start 90.08 77.5) (end 90 77.5) (width 0.5) (layer "B.Cu") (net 13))
 (segment (start 95.5 56.58) (end 92.5 59.58) (width 0.5) (layer "B.Cu") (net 13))
 (segment (start 71.5 41) (end 73 39.5) (width 0.5) (layer "B.Cu") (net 13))
 (segment (start 85.62 39.5) (end 90.12 44) (width 0.5) (layer "B.Cu") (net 13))
 (segment (start 73 39.5) (end 85.62 39.5) (width 0.5) (layer "B.Cu") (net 13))
 (segment (start 90.12 44) (end 95.5 49.38) (width 0.5) (layer "B.Cu") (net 13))
 (segment (start 71.5 79) (end 71.5 41) (width 0.5) (layer "B.Cu") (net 13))
 (segment (start 89.73 59.62) (end 92.31 59.62) (width 0.5) (layer "B.Cu") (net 13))
 (segment (start 95.5 49.38) (end 95.5 56.58) (width 0.5) (layer "B.Cu") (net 13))
 (segment (start 92.31 59.62) (end 92.35 59.58) (width 0.5) (layer "B.Cu") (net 13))
 (segment (start 85.5 82) (end 74.5 82) (width 0.5) (layer "B.Cu") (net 13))
 (segment (start 97.5 46.3) (end 97.5 64.66) (width 0.5) (layer "B.Cu") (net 11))
 (segment (start 96.5 64.66) (end 92.5 64.66) (width 0.5) (layer "B.Cu") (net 11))
 (segment (start 97.5 64.66) (end 96.5 64.66) (width 0.5) (layer "B.Cu") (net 11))
 (segment (start 95.2 44) (end 97.5 46.3) (width 0.5) (layer "B.Cu") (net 11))
 (segment (start 97.5 64.66) (end 97.5 75.16) (width 0.5) (layer "B.Cu") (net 11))
 (segment (start 97.5 75.16) (end 95.16 77.5) (width 0.5) (layer "B.Cu") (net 11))
 (segment (start 96.5 47.84) (end 96.5 58.12) (width 0.5) (layer "B.Cu") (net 12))
 (segment (start 90.5 63.5) (end 91.88 62.12) (width 0.5) (layer "B.Cu") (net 12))
 (segment (start 92.66 44) (end 96.5 47.84) (width 0.5) (layer "B.Cu") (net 12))
 (segment (start 96.5 58.12) (end 92.5 62.12) (width 0.5) (layer "B.Cu") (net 12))
 (segment (start 93.89559 65.911) (end 91.411 65.911) (width 0.5) (layer "B.Cu") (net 12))
 (segment (start 94.5 66.51541) (end 93.89559 65.911) (width 0.5) (layer "B.Cu") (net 12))
 (segment (start 91.411 65.911) (end 90.5 65) (width 0.5) (layer "B.Cu") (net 12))
 (segment (start 92.62 77.5) (end 94.5 75.62) (width 0.5) (layer "B.Cu") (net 12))
 (segment (start 94.5 75.62) (end 94.5 66.51541) (width 0.5) (layer "B.Cu") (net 12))
 (segment (start 91.88 62.12) (end 92.5 62.12) (width 0.5) (layer "B.Cu") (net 12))
 (segment (start 90.5 65) (end 90.5 63.5) (width 0.5) (layer "B.Cu") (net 12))
 (segment (start 86.73 67.74) (end 86.73 51) (width 0.5) (layer "B.Cu") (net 8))
 (segment (start 74.350854 46) (end 73.5 45.149146) (width 0.5) (layer "B.Cu") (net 8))
 (segment (start 79.25 46) (end 74.350854 46) (width 0.5) (layer "B.Cu") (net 8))
 (segment (start 86.73 51) (end 82.73 47) (width 0.5) (layer "B.Cu") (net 8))
 (segment (start 74 41.5) (end 80 41.5) (width 0.5) (layer "B.Cu") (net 8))
 (segment (start 73.5 42) (end 74 41.5) (width 0.5) (layer "B.Cu") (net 8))
 (segment (start 82.73 47) (end 80.25 47) (width 0.5) (layer "B.Cu") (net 8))
 (segment (start 80 41.5) (end 82.5 44) (width 0.5) (layer "B.Cu") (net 8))
 (segment (start 73.5 45.149146) (end 73.5 42) (width 0.5) (layer "B.Cu") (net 8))
 (segment (start 80.25 47) (end 79.25 46) (width 0.5) (layer "B.Cu") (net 8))
 (segment (start 82.46 77.5) (end 82.46 72.01) (width 0.5) (layer "B.Cu") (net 8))
 (segment (start 82.46 72.01) (end 86.73 67.74) (width 0.5) (layer "B.Cu") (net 8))
 (segment (start 87.54 75.96) (end 92.5 71) (width 0.5) (layer "B.Cu") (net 9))
 (segment (start 92.5 71) (end 92.5 69.74) (width 0.5) (layer "B.Cu") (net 9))
 (segment (start 87.54 77.5) (end 87.54 75.96) (width 0.5) (layer "B.Cu") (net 9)))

